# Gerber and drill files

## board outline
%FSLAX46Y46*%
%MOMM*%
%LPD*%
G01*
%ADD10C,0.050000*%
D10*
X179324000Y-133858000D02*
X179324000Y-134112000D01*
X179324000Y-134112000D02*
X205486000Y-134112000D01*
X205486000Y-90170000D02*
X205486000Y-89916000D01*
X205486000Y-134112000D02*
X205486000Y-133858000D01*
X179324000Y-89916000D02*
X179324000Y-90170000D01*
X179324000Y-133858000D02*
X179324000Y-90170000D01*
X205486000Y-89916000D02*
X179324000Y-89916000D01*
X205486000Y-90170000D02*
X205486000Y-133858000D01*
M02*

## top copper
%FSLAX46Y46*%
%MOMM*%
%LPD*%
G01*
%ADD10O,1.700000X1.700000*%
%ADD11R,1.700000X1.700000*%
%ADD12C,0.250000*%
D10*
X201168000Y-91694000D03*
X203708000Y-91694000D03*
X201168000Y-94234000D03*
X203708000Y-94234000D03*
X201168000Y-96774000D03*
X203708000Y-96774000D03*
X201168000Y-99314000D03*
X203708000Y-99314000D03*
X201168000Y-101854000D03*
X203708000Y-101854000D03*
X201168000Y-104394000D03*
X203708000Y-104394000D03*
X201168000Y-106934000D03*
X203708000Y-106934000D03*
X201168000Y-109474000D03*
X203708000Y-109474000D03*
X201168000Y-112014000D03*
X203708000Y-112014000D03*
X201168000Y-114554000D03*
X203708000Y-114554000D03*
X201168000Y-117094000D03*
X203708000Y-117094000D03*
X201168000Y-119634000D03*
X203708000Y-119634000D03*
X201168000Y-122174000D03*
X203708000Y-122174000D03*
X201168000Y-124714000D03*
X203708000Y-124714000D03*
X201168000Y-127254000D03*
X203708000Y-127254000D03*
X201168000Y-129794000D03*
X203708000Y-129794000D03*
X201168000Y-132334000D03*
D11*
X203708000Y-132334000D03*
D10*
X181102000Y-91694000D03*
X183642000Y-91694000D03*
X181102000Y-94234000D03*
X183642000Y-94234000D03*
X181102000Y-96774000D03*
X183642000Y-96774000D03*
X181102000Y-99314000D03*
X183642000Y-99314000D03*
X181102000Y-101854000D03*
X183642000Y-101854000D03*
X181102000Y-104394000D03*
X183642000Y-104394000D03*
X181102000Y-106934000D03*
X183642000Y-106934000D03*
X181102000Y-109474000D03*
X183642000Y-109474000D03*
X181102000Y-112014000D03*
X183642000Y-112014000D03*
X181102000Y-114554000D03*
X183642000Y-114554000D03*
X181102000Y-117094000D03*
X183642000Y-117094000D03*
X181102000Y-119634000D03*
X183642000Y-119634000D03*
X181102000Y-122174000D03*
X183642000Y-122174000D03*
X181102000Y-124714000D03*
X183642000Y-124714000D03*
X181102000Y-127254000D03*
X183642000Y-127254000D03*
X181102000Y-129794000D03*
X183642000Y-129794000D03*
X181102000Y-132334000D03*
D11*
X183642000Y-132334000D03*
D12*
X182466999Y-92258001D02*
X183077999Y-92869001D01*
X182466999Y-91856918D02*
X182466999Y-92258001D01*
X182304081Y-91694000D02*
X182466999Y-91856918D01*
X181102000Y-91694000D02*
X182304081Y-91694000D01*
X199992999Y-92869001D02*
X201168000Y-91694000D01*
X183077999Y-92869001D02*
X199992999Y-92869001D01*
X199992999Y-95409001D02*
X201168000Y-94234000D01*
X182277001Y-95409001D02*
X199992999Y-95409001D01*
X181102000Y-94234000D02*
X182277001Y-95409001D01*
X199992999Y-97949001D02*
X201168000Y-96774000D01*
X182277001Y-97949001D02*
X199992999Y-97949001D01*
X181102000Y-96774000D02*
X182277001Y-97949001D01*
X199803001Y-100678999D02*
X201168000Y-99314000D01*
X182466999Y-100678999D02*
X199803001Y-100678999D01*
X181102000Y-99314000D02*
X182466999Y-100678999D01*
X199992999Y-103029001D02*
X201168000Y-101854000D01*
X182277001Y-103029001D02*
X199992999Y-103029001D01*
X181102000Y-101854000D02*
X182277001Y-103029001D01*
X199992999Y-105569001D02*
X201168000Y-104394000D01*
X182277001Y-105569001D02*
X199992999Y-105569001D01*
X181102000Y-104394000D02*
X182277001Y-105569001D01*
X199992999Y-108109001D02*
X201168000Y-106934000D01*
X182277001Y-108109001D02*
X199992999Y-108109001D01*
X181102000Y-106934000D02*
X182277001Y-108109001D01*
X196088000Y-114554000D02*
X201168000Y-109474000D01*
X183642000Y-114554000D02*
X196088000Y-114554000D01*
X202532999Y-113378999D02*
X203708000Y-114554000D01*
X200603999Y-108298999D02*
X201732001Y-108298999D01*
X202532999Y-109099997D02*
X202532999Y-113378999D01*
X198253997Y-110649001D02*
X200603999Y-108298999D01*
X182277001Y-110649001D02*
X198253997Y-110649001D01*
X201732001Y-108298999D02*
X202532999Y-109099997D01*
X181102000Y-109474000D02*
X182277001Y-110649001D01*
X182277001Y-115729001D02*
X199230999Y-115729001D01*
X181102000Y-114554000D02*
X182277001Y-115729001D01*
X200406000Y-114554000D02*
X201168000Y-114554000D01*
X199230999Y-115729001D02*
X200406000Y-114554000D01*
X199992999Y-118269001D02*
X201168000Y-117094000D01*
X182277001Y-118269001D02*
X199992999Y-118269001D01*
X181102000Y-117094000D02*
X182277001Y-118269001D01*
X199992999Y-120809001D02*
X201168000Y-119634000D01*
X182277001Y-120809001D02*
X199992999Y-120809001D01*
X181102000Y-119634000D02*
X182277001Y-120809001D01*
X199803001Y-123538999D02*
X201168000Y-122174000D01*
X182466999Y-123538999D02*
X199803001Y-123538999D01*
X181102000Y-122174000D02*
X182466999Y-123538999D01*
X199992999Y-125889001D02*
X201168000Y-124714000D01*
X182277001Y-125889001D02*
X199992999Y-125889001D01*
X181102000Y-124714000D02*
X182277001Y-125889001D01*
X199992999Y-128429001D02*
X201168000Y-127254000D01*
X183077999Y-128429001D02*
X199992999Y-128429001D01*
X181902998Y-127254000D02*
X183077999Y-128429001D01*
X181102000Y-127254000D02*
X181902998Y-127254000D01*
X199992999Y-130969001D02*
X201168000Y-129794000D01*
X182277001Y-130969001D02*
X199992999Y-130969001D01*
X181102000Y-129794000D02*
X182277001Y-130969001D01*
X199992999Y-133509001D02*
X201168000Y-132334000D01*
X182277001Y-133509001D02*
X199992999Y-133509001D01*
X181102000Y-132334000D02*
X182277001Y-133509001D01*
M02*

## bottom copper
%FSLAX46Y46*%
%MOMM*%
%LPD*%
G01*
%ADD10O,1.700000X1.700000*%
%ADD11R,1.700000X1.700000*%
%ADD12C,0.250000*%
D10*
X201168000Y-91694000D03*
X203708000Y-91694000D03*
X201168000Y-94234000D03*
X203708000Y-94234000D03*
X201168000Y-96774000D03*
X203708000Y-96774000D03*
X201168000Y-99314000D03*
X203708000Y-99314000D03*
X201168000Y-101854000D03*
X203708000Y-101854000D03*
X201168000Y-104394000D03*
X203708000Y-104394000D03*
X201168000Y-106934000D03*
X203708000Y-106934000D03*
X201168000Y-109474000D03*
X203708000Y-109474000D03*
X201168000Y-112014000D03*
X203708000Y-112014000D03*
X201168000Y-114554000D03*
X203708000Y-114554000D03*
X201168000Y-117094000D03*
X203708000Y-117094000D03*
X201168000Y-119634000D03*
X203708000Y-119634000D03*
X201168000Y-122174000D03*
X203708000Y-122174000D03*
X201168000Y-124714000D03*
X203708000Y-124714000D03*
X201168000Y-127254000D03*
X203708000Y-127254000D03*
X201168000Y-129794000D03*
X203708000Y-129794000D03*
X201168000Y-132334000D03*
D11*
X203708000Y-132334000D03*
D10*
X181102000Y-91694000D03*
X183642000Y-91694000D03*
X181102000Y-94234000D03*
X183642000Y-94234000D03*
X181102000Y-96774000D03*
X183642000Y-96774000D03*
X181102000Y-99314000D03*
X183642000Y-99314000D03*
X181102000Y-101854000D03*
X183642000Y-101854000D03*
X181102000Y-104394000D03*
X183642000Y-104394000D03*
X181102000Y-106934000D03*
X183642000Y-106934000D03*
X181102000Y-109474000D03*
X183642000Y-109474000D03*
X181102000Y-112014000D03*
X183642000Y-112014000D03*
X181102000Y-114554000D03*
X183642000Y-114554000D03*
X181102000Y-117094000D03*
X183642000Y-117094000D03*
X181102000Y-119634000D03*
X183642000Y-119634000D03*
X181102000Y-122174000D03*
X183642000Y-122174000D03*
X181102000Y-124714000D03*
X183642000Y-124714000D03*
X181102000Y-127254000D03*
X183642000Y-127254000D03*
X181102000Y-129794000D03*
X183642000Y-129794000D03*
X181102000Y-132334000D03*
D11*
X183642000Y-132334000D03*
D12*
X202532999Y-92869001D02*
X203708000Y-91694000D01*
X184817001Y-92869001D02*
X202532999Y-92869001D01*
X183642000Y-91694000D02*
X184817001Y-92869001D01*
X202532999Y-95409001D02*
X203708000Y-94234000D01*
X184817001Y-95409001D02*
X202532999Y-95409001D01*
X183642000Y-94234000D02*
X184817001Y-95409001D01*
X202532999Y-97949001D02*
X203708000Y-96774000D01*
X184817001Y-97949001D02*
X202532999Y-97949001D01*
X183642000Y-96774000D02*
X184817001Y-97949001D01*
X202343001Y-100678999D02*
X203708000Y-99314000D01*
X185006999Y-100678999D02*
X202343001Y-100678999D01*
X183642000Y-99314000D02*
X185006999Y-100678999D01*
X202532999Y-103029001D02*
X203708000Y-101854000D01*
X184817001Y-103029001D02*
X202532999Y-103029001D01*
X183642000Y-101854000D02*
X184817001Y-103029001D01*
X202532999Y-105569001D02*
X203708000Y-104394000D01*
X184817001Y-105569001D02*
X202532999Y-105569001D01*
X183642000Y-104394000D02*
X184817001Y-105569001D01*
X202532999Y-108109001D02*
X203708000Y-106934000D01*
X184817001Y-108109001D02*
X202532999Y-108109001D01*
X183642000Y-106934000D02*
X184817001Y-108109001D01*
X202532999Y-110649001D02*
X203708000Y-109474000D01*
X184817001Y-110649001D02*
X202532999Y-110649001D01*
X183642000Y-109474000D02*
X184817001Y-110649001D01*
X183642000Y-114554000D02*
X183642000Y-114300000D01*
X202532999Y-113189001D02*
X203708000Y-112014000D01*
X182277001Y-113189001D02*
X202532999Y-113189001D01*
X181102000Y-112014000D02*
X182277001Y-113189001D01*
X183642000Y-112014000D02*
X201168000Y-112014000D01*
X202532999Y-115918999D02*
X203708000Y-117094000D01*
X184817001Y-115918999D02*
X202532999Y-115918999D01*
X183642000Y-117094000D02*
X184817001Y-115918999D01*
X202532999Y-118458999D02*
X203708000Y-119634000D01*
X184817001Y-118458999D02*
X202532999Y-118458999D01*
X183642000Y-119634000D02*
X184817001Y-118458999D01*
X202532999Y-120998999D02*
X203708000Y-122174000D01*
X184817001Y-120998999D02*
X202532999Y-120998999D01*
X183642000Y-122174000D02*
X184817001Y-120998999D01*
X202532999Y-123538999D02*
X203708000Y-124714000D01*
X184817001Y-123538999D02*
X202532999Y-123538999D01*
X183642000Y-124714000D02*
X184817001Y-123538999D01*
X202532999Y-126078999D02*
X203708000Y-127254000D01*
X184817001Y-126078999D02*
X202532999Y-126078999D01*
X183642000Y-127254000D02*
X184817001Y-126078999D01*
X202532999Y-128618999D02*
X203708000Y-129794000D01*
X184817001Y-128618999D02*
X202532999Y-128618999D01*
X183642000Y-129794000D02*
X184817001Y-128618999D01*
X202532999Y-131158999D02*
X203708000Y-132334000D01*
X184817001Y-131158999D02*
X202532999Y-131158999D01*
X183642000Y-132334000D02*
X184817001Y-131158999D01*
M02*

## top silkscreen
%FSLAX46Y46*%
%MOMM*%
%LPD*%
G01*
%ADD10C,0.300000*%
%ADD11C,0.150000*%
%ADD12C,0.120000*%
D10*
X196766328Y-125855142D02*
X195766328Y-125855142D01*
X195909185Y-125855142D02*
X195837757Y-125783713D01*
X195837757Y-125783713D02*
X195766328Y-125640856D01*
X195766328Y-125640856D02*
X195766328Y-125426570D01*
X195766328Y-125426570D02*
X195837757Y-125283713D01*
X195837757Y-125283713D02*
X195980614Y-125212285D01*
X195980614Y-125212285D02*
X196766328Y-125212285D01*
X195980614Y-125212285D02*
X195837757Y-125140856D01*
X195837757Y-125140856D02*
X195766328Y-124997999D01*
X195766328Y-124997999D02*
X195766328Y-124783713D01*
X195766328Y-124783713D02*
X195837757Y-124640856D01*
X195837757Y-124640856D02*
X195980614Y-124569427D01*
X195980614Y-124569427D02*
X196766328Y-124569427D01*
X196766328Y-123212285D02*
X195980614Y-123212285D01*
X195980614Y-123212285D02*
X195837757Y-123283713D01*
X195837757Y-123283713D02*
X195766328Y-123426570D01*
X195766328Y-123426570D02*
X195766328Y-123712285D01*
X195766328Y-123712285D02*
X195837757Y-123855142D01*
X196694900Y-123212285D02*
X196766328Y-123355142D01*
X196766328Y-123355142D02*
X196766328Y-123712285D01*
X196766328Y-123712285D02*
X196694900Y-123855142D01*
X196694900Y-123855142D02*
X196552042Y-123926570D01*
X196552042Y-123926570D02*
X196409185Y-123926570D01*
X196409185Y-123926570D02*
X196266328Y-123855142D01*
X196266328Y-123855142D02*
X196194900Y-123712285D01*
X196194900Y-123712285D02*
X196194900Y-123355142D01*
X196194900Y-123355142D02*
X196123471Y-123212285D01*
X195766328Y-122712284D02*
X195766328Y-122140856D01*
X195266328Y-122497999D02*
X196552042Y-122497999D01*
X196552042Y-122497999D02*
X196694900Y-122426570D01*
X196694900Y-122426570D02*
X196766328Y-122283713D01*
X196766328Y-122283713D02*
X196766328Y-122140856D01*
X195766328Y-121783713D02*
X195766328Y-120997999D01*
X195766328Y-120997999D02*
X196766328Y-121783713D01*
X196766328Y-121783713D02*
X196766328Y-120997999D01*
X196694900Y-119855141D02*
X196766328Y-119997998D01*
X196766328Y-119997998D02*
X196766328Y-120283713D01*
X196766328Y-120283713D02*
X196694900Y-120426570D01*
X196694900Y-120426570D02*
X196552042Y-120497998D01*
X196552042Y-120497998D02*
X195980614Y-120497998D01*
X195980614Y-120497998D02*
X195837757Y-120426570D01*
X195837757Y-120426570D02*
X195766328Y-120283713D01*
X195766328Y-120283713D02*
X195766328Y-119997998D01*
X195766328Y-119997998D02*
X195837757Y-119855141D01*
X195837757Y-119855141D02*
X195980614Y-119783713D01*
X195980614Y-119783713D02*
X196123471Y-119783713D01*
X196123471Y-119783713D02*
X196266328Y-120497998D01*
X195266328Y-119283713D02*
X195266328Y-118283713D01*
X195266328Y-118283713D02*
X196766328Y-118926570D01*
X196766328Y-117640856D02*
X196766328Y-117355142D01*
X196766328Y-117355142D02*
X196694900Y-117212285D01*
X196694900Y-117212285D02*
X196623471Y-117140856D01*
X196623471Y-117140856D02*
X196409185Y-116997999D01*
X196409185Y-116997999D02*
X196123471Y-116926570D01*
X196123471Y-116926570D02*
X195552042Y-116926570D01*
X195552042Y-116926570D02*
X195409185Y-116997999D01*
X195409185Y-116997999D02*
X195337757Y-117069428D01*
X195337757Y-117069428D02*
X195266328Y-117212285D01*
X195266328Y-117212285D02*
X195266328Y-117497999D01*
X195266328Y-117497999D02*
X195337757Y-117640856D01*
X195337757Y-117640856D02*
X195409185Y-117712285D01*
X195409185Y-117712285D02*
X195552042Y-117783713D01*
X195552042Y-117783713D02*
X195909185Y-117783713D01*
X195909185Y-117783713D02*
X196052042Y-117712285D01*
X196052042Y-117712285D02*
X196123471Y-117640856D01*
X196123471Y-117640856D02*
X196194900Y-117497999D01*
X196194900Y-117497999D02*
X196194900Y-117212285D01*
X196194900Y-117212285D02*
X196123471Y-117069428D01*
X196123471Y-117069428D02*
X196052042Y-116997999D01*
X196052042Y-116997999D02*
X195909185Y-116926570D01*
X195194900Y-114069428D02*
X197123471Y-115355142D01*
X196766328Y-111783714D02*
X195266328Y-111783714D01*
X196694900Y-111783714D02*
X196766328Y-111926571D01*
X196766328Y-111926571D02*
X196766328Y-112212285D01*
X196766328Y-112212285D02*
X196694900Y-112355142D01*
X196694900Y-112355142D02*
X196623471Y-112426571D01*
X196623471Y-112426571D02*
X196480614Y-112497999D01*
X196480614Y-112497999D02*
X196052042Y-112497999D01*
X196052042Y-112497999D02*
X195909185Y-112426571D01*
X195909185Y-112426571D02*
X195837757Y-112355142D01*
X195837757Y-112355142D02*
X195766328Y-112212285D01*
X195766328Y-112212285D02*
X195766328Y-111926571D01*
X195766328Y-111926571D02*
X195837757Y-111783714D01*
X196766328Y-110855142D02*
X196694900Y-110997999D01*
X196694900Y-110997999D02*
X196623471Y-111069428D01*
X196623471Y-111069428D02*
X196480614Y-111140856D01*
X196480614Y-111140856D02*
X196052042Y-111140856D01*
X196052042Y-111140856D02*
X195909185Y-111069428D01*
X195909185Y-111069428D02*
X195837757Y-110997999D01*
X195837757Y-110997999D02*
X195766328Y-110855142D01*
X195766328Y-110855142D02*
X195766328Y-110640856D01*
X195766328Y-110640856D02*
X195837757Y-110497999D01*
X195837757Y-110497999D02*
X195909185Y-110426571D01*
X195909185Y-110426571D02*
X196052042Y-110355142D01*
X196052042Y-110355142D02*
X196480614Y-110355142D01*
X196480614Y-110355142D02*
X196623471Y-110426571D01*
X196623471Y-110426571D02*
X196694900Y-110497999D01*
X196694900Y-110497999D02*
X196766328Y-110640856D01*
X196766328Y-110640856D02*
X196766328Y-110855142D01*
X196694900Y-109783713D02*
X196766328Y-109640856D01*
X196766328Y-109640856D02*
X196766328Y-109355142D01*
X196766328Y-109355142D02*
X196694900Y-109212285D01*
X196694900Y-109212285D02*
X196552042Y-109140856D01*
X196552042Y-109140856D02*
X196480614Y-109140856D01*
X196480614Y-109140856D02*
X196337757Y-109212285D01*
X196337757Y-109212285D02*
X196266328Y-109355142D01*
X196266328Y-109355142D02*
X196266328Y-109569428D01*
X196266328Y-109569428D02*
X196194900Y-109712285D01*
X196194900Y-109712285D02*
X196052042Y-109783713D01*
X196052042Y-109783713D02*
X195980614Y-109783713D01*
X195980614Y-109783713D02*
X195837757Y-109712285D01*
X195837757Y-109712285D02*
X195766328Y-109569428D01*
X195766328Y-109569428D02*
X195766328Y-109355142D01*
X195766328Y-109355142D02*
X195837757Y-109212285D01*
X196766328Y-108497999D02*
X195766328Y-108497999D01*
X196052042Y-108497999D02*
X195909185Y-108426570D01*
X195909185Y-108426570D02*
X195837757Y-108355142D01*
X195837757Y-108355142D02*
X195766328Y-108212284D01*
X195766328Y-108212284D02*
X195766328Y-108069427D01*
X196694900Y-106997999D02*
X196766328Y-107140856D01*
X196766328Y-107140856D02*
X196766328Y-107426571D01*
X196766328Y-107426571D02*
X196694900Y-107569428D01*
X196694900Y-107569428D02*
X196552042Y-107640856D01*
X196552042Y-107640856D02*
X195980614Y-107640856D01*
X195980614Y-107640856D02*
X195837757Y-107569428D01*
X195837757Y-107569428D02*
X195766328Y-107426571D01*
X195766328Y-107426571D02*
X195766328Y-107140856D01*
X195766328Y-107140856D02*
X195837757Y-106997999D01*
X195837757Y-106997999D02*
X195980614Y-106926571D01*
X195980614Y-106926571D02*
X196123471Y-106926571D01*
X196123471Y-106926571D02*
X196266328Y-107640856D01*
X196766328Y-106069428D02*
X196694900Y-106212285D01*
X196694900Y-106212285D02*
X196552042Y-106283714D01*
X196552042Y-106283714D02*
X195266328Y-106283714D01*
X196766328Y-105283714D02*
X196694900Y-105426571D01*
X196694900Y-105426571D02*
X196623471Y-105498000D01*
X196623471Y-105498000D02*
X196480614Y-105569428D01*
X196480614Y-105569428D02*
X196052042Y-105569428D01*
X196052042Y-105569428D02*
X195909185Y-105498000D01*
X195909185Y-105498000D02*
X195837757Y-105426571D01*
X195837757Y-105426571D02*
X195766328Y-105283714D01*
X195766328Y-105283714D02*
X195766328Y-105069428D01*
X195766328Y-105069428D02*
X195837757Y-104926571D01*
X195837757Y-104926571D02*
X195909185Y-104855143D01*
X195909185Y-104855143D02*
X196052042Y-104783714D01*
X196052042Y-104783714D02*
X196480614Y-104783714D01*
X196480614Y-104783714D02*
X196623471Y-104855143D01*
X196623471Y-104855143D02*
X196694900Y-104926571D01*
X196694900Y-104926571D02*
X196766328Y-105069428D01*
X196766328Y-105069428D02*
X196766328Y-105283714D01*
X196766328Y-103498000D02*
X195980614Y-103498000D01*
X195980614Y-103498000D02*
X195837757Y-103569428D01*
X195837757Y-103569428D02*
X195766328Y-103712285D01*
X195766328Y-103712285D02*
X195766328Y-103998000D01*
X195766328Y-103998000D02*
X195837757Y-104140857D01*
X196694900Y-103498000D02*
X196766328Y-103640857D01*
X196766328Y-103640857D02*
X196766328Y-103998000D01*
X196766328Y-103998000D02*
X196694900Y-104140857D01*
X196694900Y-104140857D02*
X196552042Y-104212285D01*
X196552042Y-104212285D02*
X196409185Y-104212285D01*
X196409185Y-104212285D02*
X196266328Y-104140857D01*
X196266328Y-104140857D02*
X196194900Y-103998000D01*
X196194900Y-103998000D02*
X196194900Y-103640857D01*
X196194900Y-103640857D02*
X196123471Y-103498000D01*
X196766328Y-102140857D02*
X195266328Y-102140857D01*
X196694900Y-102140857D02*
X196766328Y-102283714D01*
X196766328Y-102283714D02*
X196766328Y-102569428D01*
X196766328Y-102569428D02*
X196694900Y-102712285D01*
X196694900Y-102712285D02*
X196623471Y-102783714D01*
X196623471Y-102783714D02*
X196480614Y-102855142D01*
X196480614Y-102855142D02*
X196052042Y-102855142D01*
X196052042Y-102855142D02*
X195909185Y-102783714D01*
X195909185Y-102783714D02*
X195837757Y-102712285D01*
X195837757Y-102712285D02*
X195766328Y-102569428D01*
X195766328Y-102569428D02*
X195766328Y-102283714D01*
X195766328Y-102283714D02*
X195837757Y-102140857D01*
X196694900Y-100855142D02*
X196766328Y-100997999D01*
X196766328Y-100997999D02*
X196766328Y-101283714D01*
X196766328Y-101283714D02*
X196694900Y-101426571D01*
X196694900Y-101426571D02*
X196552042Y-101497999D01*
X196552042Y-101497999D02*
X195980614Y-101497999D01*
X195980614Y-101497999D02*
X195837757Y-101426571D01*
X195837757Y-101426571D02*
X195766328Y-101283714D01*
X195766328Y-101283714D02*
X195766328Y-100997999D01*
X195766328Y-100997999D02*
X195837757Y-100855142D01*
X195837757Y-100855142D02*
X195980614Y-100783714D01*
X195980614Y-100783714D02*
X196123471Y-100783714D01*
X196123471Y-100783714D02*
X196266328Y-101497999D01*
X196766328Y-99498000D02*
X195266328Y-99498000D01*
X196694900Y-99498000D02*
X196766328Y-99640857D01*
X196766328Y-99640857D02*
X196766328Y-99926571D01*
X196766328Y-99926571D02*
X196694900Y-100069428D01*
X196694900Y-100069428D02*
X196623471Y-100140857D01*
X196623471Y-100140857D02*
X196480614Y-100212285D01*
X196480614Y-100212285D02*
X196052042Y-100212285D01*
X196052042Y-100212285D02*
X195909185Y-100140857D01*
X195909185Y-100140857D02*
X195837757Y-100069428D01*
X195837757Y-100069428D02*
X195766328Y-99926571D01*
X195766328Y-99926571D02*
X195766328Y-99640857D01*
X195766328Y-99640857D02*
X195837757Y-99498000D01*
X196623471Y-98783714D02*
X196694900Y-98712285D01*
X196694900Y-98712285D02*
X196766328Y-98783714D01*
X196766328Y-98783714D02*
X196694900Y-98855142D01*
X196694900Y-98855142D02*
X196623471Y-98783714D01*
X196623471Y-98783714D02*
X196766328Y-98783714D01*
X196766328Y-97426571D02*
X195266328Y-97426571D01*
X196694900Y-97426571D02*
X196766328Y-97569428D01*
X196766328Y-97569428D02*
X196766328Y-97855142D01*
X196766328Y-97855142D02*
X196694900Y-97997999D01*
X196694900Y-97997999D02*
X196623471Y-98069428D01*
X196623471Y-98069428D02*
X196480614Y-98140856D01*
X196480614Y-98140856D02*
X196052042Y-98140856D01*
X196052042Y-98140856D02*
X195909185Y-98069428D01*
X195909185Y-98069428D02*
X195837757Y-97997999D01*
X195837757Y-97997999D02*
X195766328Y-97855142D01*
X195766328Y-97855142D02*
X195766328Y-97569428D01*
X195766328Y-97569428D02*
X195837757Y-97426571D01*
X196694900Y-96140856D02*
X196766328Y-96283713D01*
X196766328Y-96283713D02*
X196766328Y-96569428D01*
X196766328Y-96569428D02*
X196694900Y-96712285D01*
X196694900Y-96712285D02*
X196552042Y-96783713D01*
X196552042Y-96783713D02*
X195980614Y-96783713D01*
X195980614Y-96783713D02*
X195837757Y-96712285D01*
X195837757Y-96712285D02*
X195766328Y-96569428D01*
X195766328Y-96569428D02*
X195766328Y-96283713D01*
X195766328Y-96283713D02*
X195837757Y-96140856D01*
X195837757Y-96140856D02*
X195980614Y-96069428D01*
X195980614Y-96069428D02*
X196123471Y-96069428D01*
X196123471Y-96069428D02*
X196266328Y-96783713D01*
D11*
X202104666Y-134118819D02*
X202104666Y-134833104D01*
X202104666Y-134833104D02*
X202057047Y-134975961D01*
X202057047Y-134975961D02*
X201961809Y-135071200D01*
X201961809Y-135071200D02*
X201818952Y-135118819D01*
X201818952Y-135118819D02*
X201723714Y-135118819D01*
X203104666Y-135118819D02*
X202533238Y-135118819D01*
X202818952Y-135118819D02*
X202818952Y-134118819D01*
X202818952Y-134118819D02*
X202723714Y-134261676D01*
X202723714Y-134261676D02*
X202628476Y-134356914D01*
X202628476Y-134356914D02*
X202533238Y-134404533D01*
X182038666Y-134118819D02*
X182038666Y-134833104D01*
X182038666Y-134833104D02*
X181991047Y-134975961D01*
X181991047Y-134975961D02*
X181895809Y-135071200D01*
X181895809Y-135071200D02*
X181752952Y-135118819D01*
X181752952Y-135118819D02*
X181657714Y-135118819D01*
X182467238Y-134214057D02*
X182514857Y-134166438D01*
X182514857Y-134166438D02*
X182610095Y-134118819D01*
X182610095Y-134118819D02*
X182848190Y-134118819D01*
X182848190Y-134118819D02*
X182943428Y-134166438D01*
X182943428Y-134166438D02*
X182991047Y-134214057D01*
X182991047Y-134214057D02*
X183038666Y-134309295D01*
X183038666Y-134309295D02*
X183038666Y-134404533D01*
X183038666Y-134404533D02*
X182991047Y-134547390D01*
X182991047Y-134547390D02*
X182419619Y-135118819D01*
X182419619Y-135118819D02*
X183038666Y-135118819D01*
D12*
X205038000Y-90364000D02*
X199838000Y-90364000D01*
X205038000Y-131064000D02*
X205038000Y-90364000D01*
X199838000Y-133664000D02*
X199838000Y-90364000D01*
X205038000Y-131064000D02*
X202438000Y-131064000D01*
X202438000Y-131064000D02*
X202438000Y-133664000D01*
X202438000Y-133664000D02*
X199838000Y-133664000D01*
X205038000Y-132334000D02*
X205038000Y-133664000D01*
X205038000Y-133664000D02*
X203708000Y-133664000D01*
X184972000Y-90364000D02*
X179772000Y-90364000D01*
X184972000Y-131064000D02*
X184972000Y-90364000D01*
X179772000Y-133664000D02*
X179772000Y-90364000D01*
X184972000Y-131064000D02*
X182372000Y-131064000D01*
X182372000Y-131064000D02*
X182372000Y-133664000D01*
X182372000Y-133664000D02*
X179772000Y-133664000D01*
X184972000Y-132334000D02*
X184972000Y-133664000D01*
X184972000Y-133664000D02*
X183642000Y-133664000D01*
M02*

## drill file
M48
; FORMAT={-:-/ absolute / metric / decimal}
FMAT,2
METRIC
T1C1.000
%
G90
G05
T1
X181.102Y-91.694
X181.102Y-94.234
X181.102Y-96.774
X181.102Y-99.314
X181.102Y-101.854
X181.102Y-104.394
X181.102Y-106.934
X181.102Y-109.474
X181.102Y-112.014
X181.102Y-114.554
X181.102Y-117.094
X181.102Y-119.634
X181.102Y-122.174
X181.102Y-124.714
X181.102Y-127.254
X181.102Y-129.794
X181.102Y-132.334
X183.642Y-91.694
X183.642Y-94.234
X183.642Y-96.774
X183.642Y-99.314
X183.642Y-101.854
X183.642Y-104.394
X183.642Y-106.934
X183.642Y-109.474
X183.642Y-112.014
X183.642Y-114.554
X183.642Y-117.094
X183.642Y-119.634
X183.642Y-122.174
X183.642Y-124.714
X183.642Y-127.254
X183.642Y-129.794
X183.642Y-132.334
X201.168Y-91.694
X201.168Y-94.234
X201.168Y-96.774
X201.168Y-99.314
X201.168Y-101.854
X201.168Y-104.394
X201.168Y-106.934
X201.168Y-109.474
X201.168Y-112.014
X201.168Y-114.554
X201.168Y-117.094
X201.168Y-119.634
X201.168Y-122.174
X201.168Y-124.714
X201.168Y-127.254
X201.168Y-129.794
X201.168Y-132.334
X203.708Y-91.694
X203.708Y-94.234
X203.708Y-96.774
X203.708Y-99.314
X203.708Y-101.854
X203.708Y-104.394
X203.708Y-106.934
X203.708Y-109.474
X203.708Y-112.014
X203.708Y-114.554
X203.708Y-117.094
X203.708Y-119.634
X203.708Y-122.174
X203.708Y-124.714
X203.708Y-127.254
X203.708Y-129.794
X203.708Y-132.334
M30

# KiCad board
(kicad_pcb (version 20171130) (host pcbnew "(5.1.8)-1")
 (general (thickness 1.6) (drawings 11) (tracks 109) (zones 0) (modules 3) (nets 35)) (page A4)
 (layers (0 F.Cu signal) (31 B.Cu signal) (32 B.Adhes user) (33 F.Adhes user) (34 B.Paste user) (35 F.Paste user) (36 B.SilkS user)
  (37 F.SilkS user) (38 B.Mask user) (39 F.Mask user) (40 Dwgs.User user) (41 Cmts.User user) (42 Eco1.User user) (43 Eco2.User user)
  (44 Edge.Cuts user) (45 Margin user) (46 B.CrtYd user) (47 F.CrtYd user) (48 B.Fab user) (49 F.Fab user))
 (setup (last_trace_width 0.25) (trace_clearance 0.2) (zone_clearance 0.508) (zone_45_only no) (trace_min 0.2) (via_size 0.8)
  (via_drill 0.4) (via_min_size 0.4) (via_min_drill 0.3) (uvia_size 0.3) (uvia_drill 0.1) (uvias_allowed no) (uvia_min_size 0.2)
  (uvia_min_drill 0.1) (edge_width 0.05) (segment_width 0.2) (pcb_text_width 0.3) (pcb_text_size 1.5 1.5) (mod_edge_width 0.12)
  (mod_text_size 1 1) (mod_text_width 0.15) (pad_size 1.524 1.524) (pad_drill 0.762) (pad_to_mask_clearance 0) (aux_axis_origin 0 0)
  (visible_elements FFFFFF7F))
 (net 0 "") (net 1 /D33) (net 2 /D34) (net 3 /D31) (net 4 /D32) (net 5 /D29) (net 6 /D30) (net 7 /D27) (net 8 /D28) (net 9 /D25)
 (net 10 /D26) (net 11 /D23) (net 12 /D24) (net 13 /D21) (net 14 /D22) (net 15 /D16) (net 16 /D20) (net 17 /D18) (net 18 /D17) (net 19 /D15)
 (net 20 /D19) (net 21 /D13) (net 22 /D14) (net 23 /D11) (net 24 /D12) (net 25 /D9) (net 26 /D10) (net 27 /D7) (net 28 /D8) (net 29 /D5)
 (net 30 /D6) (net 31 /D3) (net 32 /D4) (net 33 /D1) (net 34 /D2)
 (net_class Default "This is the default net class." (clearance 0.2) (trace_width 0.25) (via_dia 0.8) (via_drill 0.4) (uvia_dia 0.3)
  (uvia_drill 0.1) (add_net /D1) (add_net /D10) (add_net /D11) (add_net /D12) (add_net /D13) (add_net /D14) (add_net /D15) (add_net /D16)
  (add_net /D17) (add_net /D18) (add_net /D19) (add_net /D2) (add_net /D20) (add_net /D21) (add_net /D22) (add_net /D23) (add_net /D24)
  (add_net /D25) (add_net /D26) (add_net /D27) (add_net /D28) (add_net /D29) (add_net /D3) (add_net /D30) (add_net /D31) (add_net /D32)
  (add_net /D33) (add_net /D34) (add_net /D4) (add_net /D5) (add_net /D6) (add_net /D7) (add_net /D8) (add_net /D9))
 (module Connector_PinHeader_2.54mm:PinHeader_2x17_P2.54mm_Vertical (layer F.Cu) (at 203.708 132.334 180)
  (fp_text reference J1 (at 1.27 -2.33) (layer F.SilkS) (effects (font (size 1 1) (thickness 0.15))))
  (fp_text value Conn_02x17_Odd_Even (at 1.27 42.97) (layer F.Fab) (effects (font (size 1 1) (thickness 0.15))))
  (fp_line (start -1.33 41.97) (end 3.87 41.97) (layer F.SilkS) (width 0.12))
  (fp_line (start -1.33 1.27) (end -1.33 41.97) (layer F.SilkS) (width 0.12))
  (fp_line (start 3.87 -1.33) (end 3.87 41.97) (layer F.SilkS) (width 0.12))
  (fp_line (start -1.33 1.27) (end 1.27 1.27) (layer F.SilkS) (width 0.12))
  (fp_line (start 1.27 1.27) (end 1.27 -1.33) (layer F.SilkS) (width 0.12))
  (fp_line (start 1.27 -1.33) (end 3.87 -1.33) (layer F.SilkS) (width 0.12))
  (fp_line (start -1.33 0) (end -1.33 -1.33) (layer F.SilkS) (width 0.12))
  (fp_line (start -1.33 -1.33) (end 0 -1.33) (layer F.SilkS) (width 0.12))
  (pad 34 thru_hole oval (at 2.54 40.64 180) (size 1.7 1.7) (drill 1) (layers *.Cu *.Mask) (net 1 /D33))
  (pad 33 thru_hole oval (at 0 40.64 180) (size 1.7 1.7) (drill 1) (layers *.Cu *.Mask) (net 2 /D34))
  (pad 32 thru_hole oval (at 2.54 38.1 180) (size 1.7 1.7) (drill 1) (layers *.Cu *.Mask) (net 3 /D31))
  (pad 31 thru_hole oval (at 0 38.1 180) (size 1.7 1.7) (drill 1) (layers *.Cu *.Mask) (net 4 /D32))
  (pad 30 thru_hole oval (at 2.54 35.56 180) (size 1.7 1.7) (drill 1) (layers *.Cu *.Mask) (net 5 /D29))
  (pad 29 thru_hole oval (at 0 35.56 180) (size 1.7 1.7) (drill 1) (layers *.Cu *.Mask) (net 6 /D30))
  (pad 28 thru_hole oval (at 2.54 33.02 180) (size 1.7 1.7) (drill 1) (layers *.Cu *.Mask) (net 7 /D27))
  (pad 27 thru_hole oval (at 0 33.02 180) (size 1.7 1.7) (drill 1) (layers *.Cu *.Mask) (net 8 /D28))
  (pad 26 thru_hole oval (at 2.54 30.48 180) (size 1.7 1.7) (drill 1) (layers *.Cu *.Mask) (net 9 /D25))
  (pad 25 thru_hole oval (at 0 30.48 180) (size 1.7 1.7) (drill 1) (layers *.Cu *.Mask) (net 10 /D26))
  (pad 24 thru_hole oval (at 2.54 27.94 180) (size 1.7 1.7) (drill 1) (layers *.Cu *.Mask) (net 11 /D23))
  (pad 23 thru_hole oval (at 0 27.94 180) (size 1.7 1.7) (drill 1) (layers *.Cu *.Mask) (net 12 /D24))
  (pad 22 thru_hole oval (at 2.54 25.4 180) (size 1.7 1.7) (drill 1) (layers *.Cu *.Mask) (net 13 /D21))
  (pad 21 thru_hole oval (at 0 25.4 180) (size 1.7 1.7) (drill 1) (layers *.Cu *.Mask) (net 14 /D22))
  (pad 20 thru_hole oval (at 2.54 22.86 180) (size 1.7 1.7) (drill 1) (layers *.Cu *.Mask) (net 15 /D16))
  (pad 19 thru_hole oval (at 0 22.86 180) (size 1.7 1.7) (drill 1) (layers *.Cu *.Mask) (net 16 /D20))
  (pad 18 thru_hole oval (at 2.54 20.32 180) (size 1.7 1.7) (drill 1) (layers *.Cu *.Mask) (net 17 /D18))
  (pad 17 thru_hole oval (at 0 20.32 180) (size 1.7 1.7) (drill 1) (layers *.Cu *.Mask) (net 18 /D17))
  (pad 16 thru_hole oval (at 2.54 17.78 180) (size 1.7 1.7) (drill 1) (layers *.Cu *.Mask) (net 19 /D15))
  (pad 15 thru_hole oval (at 0 17.78 180) (size 1.7 1.7) (drill 1) (layers *.Cu *.Mask) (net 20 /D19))
  (pad 14 thru_hole oval (at 2.54 15.24 180) (size 1.7 1.7) (drill 1) (layers *.Cu *.Mask) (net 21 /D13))
  (pad 13 thru_hole oval (at 0 15.24 180) (size 1.7 1.7) (drill 1) (layers *.Cu *.Mask) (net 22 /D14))
  (pad 12 thru_hole oval (at 2.54 12.7 180) (size 1.7 1.7) (drill 1) (layers *.Cu *.Mask) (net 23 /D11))
  (pad 11 thru_hole oval (at 0 12.7 180) (size 1.7 1.7) (drill 1) (layers *.Cu *.Mask) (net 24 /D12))
  (pad 10 thru_hole oval (at 2.54 10.16 180) (size 1.7 1.7) (drill 1) (layers *.Cu *.Mask) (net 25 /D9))
  (pad 9 thru_hole oval (at 0 10.16 180) (size 1.7 1.7) (drill 1) (layers *.Cu *.Mask) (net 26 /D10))
  (pad 8 thru_hole oval (at 2.54 7.62 180) (size 1.7 1.7) (drill 1) (layers *.Cu *.Mask) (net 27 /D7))
  (pad 7 thru_hole oval (at 0 7.62 180) (size 1.7 1.7) (drill 1) (layers *.Cu *.Mask) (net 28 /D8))
  (pad 6 thru_hole oval (at 2.54 5.08 180) (size 1.7 1.7) (drill 1) (layers *.Cu *.Mask) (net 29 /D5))
  (pad 5 thru_hole oval (at 0 5.08 180) (size 1.7 1.7) (drill 1) (layers *.Cu *.Mask) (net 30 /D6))
  (pad 4 thru_hole oval (at 2.54 2.54 180) (size 1.7 1.7) (drill 1) (layers *.Cu *.Mask) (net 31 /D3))
  (pad 3 thru_hole oval (at 0 2.54 180) (size 1.7 1.7) (drill 1) (layers *.Cu *.Mask) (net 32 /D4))
  (pad 2 thru_hole oval (at 2.54 0 180) (size 1.7 1.7) (drill 1) (layers *.Cu *.Mask) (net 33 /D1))
  (pad 1 thru_hole rect (at 0 0 180) (size 1.7 1.7) (drill 1) (layers *.Cu *.Mask) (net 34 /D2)))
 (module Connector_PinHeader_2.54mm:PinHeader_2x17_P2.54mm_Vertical (layer F.Cu) (at 183.642 132.334 180)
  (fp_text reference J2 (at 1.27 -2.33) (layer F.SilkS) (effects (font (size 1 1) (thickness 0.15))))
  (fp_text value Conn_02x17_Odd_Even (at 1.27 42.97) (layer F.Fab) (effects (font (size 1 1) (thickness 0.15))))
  (fp_line (start -1.33 41.97) (end 3.87 41.97) (layer F.SilkS) (width 0.12))
  (fp_line (start -1.33 1.27) (end -1.33 41.97) (layer F.SilkS) (width 0.12))
  (fp_line (start 3.87 -1.33) (end 3.87 41.97) (layer F.SilkS) (width 0.12))
  (fp_line (start -1.33 1.27) (end 1.27 1.27) (layer F.SilkS) (width 0.12))
  (fp_line (start 1.27 1.27) (end 1.27 -1.33) (layer F.SilkS) (width 0.12))
  (fp_line (start 1.27 -1.33) (end 3.87 -1.33) (layer F.SilkS) (width 0.12))
  (fp_line (start -1.33 0) (end -1.33 -1.33) (layer F.SilkS) (width 0.12))
  (fp_line (start -1.33 -1.33) (end 0 -1.33) (layer F.SilkS) (width 0.12))
  (pad 34 thru_hole oval (at 2.54 40.64 180) (size 1.7 1.7) (drill 1) (layers *.Cu *.Mask) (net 1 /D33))
  (pad 33 thru_hole oval (at 0 40.64 180) (size 1.7 1.7) (drill 1) (layers *.Cu *.Mask) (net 2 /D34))
  (pad 32 thru_hole oval (at 2.54 38.1 180) (size 1.7 1.7) (drill 1) (layers *.Cu *.Mask) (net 3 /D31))
  (pad 31 thru_hole oval (at 0 38.1 180) (size 1.7 1.7) (drill 1) (layers *.Cu *.Mask) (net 4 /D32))
  (pad 30 thru_hole oval (at 2.54 35.56 180) (size 1.7 1.7) (drill 1) (layers *.Cu *.Mask) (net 5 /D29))
  (pad 29 thru_hole oval (at 0 35.56 180) (size 1.7 1.7) (drill 1) (layers *.Cu *.Mask) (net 6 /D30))
  (pad 28 thru_hole oval (at 2.54 33.02 180) (size 1.7 1.7) (drill 1) (layers *.Cu *.Mask) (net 7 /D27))
  (pad 27 thru_hole oval (at 0 33.02 180) (size 1.7 1.7) (drill 1) (layers *.Cu *.Mask) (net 8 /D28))
  (pad 26 thru_hole oval (at 2.54 30.48 180) (size 1.7 1.7) (drill 1) (layers *.Cu *.Mask) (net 9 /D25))
  (pad 25 thru_hole oval (at 0 30.48 180) (size 1.7 1.7) (drill 1) (layers *.Cu *.Mask) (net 10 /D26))
  (pad 24 thru_hole oval (at 2.54 27.94 180) (size 1.7 1.7) (drill 1) (layers *.Cu *.Mask) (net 11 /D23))
  (pad 23 thru_hole oval (at 0 27.94 180) (size 1.7 1.7) (drill 1) (layers *.Cu *.Mask) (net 12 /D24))
  (pad 22 thru_hole oval (at 2.54 25.4 180) (size 1.7 1.7) (drill 1) (layers *.Cu *.Mask) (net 13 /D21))
  (pad 21 thru_hole oval (at 0 25.4 180) (size 1.7 1.7) (drill 1) (layers *.Cu *.Mask) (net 14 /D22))
  (pad 20 thru_hole oval (at 2.54 22.86 180) (size 1.7 1.7) (drill 1) (layers *.Cu *.Mask) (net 20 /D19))
  (pad 19 thru_hole oval (at 0 22.86 180) (size 1.7 1.7) (drill 1) (layers *.Cu *.Mask) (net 16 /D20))
  (pad 18 thru_hole oval (at 2.54 20.32 180) (size 1.7 1.7) (drill 1) (layers *.Cu *.Mask) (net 18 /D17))
  (pad 17 thru_hole oval (at 0 20.32 180) (size 1.7 1.7) (drill 1) (layers *.Cu *.Mask) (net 17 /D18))
  (pad 16 thru_hole oval (at 2.54 17.78 180) (size 1.7 1.7) (drill 1) (layers *.Cu *.Mask) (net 19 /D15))
  (pad 15 thru_hole oval (at 0 17.78 180) (size 1.7 1.7) (drill 1) (layers *.Cu *.Mask) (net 15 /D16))
  (pad 14 thru_hole oval (at 2.54 15.24 180) (size 1.7 1.7) (drill 1) (layers *.Cu *.Mask) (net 21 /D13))
  (pad 13 thru_hole oval (at 0 15.24 180) (size 1.7 1.7) (drill 1) (layers *.Cu *.Mask) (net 22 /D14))
  (pad 12 thru_hole oval (at 2.54 12.7 180) (size 1.7 1.7) (drill 1) (layers *.Cu *.Mask) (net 23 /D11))
  (pad 11 thru_hole oval (at 0 12.7 180) (size 1.7 1.7) (drill 1) (layers *.Cu *.Mask) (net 24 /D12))
  (pad 10 thru_hole oval (at 2.54 10.16 180) (size 1.7 1.7) (drill 1) (layers *.Cu *.Mask) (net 25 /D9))
  (pad 9 thru_hole oval (at 0 10.16 180) (size 1.7 1.7) (drill 1) (layers *.Cu *.Mask) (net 26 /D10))
  (pad 8 thru_hole oval (at 2.54 7.62 180) (size 1.7 1.7) (drill 1) (layers *.Cu *.Mask) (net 27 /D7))
  (pad 7 thru_hole oval (at 0 7.62 180) (size 1.7 1.7) (drill 1) (layers *.Cu *.Mask) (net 28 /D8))
  (pad 6 thru_hole oval (at 2.54 5.08 180) (size 1.7 1.7) (drill 1) (layers *.Cu *.Mask) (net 29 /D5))
  (pad 5 thru_hole oval (at 0 5.08 180) (size 1.7 1.7) (drill 1) (layers *.Cu *.Mask) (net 30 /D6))
  (pad 4 thru_hole oval (at 2.54 2.54 180) (size 1.7 1.7) (drill 1) (layers *.Cu *.Mask) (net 31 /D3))
  (pad 3 thru_hole oval (at 0 2.54 180) (size 1.7 1.7) (drill 1) (layers *.Cu *.Mask) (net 32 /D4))
  (pad 2 thru_hole oval (at 2.54 0 180) (size 1.7 1.7) (drill 1) (layers *.Cu *.Mask) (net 33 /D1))
  (pad 1 thru_hole rect (at 0 0 180) (size 1.7 1.7) (drill 1) (layers *.Cu *.Mask) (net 34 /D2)))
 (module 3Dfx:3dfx (layer B.Cu) (at 192.278 112.522 270)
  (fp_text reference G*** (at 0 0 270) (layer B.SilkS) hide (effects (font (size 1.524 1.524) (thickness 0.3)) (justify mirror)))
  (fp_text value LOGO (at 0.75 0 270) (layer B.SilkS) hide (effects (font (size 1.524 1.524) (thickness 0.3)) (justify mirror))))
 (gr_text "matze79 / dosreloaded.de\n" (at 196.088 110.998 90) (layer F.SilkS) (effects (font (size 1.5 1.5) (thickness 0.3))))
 (gr_line (start 179.324 133.858) (end 179.324 134.112) (layer Edge.Cuts) (width 0.05))
 (gr_line (start 179.324 134.112) (end 205.486 134.112) (layer Edge.Cuts) (width 0.05))
 (gr_line (start 205.486 90.17) (end 205.486 89.916) (layer Edge.Cuts) (width 0.05))
 (gr_line (start 205.486 134.112) (end 205.486 133.858) (layer Edge.Cuts) (width 0.05))
 (gr_line (start 179.324 89.916) (end 179.324 90.17) (layer Edge.Cuts) (width 0.05))
 (gr_line (start 179.324 133.858) (end 179.324 90.17) (layer Edge.Cuts) (width 0.05))
 (gr_line (start 205.486 89.916) (end 179.324 89.916) (layer Edge.Cuts) (width 0.05))
 (gr_line (start 205.486 90.17) (end 205.486 133.858) (layer Edge.Cuts) (width 0.05))
 (segment (start 202.532999 92.869001) (end 203.708 91.694) (width 0.25) (layer B.Cu) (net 2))
 (segment (start 184.817001 92.869001) (end 202.532999 92.869001) (width 0.25) (layer B.Cu) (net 2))
 (segment (start 183.642 91.694) (end 184.817001 92.869001) (width 0.25) (layer B.Cu) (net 2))
 (segment (start 182.466999 92.258001) (end 183.077999 92.869001) (width 0.25) (layer F.Cu) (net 1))
 (segment (start 182.466999 91.856918) (end 182.466999 92.258001) (width 0.25) (layer F.Cu) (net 1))
 (segment (start 182.304081 91.694) (end 182.466999 91.856918) (width 0.25) (layer F.Cu) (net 1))
 (segment (start 181.102 91.694) (end 182.304081 91.694) (width 0.25) (layer F.Cu) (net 1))
 (segment (start 199.992999 92.869001) (end 201.168 91.694) (width 0.25) (layer F.Cu) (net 1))
 (segment (start 183.077999 92.869001) (end 199.992999 92.869001) (width 0.25) (layer F.Cu) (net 1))
 (segment (start 202.532999 95.409001) (end 203.708 94.234) (width 0.25) (layer B.Cu) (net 4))
 (segment (start 184.817001 95.409001) (end 202.532999 95.409001) (width 0.25) (layer B.Cu) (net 4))
 (segment (start 183.642 94.234) (end 184.817001 95.409001) (width 0.25) (layer B.Cu) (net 4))
 (segment (start 199.992999 95.409001) (end 201.168 94.234) (width 0.25) (layer F.Cu) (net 3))
 (segment (start 182.277001 95.409001) (end 199.992999 95.409001) (width 0.25) (layer F.Cu) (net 3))
 (segment (start 181.102 94.234) (end 182.277001 95.409001) (width 0.25) (layer F.Cu) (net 3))
 (segment (start 202.532999 97.949001) (end 203.708 96.774) (width 0.25) (layer B.Cu) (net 6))
 (segment (start 184.817001 97.949001) (end 202.532999 97.949001) (width 0.25) (layer B.Cu) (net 6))
 (segment (start 183.642 96.774) (end 184.817001 97.949001) (width 0.25) (layer B.Cu) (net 6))
 (segment (start 199.992999 97.949001) (end 201.168 96.774) (width 0.25) (layer F.Cu) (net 5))
 (segment (start 182.277001 97.949001) (end 199.992999 97.949001) (width 0.25) (layer F.Cu) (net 5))
 (segment (start 181.102 96.774) (end 182.277001 97.949001) (width 0.25) (layer F.Cu) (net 5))
 (segment (start 202.343001 100.678999) (end 203.708 99.314) (width 0.25) (layer B.Cu) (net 8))
 (segment (start 185.006999 100.678999) (end 202.343001 100.678999) (width 0.25) (layer B.Cu) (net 8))
 (segment (start 183.642 99.314) (end 185.006999 100.678999) (width 0.25) (layer B.Cu) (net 8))
 (segment (start 199.803001 100.678999) (end 201.168 99.314) (width 0.25) (layer F.Cu) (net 7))
 (segment (start 182.466999 100.678999) (end 199.803001 100.678999) (width 0.25) (layer F.Cu) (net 7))
 (segment (start 181.102 99.314) (end 182.466999 100.678999) (width 0.25) (layer F.Cu) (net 7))
 (segment (start 202.532999 103.029001) (end 203.708 101.854) (width 0.25) (layer B.Cu) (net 10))
 (segment (start 184.817001 103.029001) (end 202.532999 103.029001) (width 0.25) (layer B.Cu) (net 10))
 (segment (start 183.642 101.854) (end 184.817001 103.029001) (width 0.25) (layer B.Cu) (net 10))
 (segment (start 199.992999 103.029001) (end 201.168 101.854) (width 0.25) (layer F.Cu) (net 9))
 (segment (start 182.277001 103.029001) (end 199.992999 103.029001) (width 0.25) (layer F.Cu) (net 9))
 (segment (start 181.102 101.854) (end 182.277001 103.029001) (width 0.25) (layer F.Cu) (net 9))
 (segment (start 202.532999 105.569001) (end 203.708 104.394) (width 0.25) (layer B.Cu) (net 12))
 (segment (start 184.817001 105.569001) (end 202.532999 105.569001) (width 0.25) (layer B.Cu) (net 12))
 (segment (start 183.642 104.394) (end 184.817001 105.569001) (width 0.25) (layer B.Cu) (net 12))
 (segment (start 199.992999 105.569001) (end 201.168 104.394) (width 0.25) (layer F.Cu) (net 11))
 (segment (start 182.277001 105.569001) (end 199.992999 105.569001) (width 0.25) (layer F.Cu) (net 11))
 (segment (start 181.102 104.394) (end 182.277001 105.569001) (width 0.25) (layer F.Cu) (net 11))
 (segment (start 202.532999 108.109001) (end 203.708 106.934) (width 0.25) (layer B.Cu) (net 14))
 (segment (start 184.817001 108.109001) (end 202.532999 108.109001) (width 0.25) (layer B.Cu) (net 14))
 (segment (start 183.642 106.934) (end 184.817001 108.109001) (width 0.25) (layer B.Cu) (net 14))
 (segment (start 199.992999 108.109001) (end 201.168 106.934) (width 0.25) (layer F.Cu) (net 13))
 (segment (start 182.277001 108.109001) (end 199.992999 108.109001) (width 0.25) (layer F.Cu) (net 13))
 (segment (start 181.102 106.934) (end 182.277001 108.109001) (width 0.25) (layer F.Cu) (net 13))
 (segment (start 202.532999 110.649001) (end 203.708 109.474) (width 0.25) (layer B.Cu) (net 16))
 (segment (start 184.817001 110.649001) (end 202.532999 110.649001) (width 0.25) (layer B.Cu) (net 16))
 (segment (start 183.642 109.474) (end 184.817001 110.649001) (width 0.25) (layer B.Cu) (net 16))
 (segment (start 183.642 114.554) (end 183.642 114.3) (width 0.25) (layer B.Cu) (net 15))
 (segment (start 196.088 114.554) (end 201.168 109.474) (width 0.25) (layer F.Cu) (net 15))
 (segment (start 183.642 114.554) (end 196.088 114.554) (width 0.25) (layer F.Cu) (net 15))
 (segment (start 202.532999 113.189001) (end 203.708 112.014) (width 0.25) (layer B.Cu) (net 18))
 (segment (start 182.277001 113.189001) (end 202.532999 113.189001) (width 0.25) (layer B.Cu) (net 18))
 (segment (start 181.102 112.014) (end 182.277001 113.189001) (width 0.25) (layer B.Cu) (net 18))
 (segment (start 183.642 112.014) (end 201.168 112.014) (width 0.25) (layer B.Cu) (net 17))
 (segment (start 202.532999 113.378999) (end 203.708 114.554) (width 0.25) (layer F.Cu) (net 20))
 (segment (start 200.603999 108.298999) (end 201.732001 108.298999) (width 0.25) (layer F.Cu) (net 20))
 (segment (start 202.532999 109.099997) (end 202.532999 113.378999) (width 0.25) (layer F.Cu) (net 20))
 (segment (start 198.253997 110.649001) (end 200.603999 108.298999) (width 0.25) (layer F.Cu) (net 20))
 (segment (start 182.277001 110.649001) (end 198.253997 110.649001) (width 0.25) (layer F.Cu) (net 20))
 (segment (start 201.732001 108.298999) (end 202.532999 109.099997) (width 0.25) (layer F.Cu) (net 20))
 (segment (start 181.102 109.474) (end 182.277001 110.649001) (width 0.25) (layer F.Cu) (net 20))
 (segment (start 182.277001 115.729001) (end 199.230999 115.729001) (width 0.25) (layer F.Cu) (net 19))
 (segment (start 181.102 114.554) (end 182.277001 115.729001) (width 0.25) (layer F.Cu) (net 19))
 (segment (start 200.406 114.554) (end 201.168 114.554) (width 0.25) (layer F.Cu) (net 19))
 (segment (start 199.230999 115.729001) (end 200.406 114.554) (width 0.25) (layer F.Cu) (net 19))
 (segment (start 202.532999 115.918999) (end 203.708 117.094) (width 0.25) (layer B.Cu) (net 22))
 (segment (start 184.817001 115.918999) (end 202.532999 115.918999) (width 0.25) (layer B.Cu) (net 22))
 (segment (start 183.642 117.094) (end 184.817001 115.918999) (width 0.25) (layer B.Cu) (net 22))
 (segment (start 199.992999 118.269001) (end 201.168 117.094) (width 0.25) (layer F.Cu) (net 21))
 (segment (start 182.277001 118.269001) (end 199.992999 118.269001) (width 0.25) (layer F.Cu) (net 21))
 (segment (start 181.102 117.094) (end 182.277001 118.269001) (width 0.25) (layer F.Cu) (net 21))
 (segment (start 202.532999 118.458999) (end 203.708 119.634) (width 0.25) (layer B.Cu) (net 24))
 (segment (start 184.817001 118.458999) (end 202.532999 118.458999) (width 0.25) (layer B.Cu) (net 24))
 (segment (start 183.642 119.634) (end 184.817001 118.458999) (width 0.25) (layer B.Cu) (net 24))
 (segment (start 199.992999 120.809001) (end 201.168 119.634) (width 0.25) (layer F.Cu) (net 23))
 (segment (start 182.277001 120.809001) (end 199.992999 120.809001) (width 0.25) (layer F.Cu) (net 23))
 (segment (start 181.102 119.634) (end 182.277001 120.809001) (width 0.25) (layer F.Cu) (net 23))
 (segment (start 202.532999 120.998999) (end 203.708 122.174) (width 0.25) (layer B.Cu) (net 26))
 (segment (start 184.817001 120.998999) (end 202.532999 120.998999) (width 0.25) (layer B.Cu) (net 26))
 (segment (start 183.642 122.174) (end 184.817001 120.998999) (width 0.25) (layer B.Cu) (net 26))
 (segment (start 199.803001 123.538999) (end 201.168 122.174) (width 0.25) (layer F.Cu) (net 25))
 (segment (start 182.466999 123.538999) (end 199.803001 123.538999) (width 0.25) (layer F.Cu) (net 25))
 (segment (start 181.102 122.174) (end 182.466999 123.538999) (width 0.25) (layer F.Cu) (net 25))
 (segment (start 202.532999 123.538999) (end 203.708 124.714) (width 0.25) (layer B.Cu) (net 28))
 (segment (start 184.817001 123.538999) (end 202.532999 123.538999) (width 0.25) (layer B.Cu) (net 28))
 (segment (start 183.642 124.714) (end 184.817001 123.538999) (width 0.25) (layer B.Cu) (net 28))
 (segment (start 199.992999 125.889001) (end 201.168 124.714) (width 0.25) (layer F.Cu) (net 27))
 (segment (start 182.277001 125.889001) (end 199.992999 125.889001) (width 0.25) (layer F.Cu) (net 27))
 (segment (start 181.102 124.714) (end 182.277001 125.889001) (width 0.25) (layer F.Cu) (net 27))
 (segment (start 202.532999 126.078999) (end 203.708 127.254) (width 0.25) (layer B.Cu) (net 30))
 (segment (start 184.817001 126.078999) (end 202.532999 126.078999) (width 0.25) (layer B.Cu) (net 30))
 (segment (start 183.642 127.254) (end 184.817001 126.078999) (width 0.25) (layer B.Cu) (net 30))
 (segment (start 199.992999 128.429001) (end 201.168 127.254) (width 0.25) (layer F.Cu) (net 29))
 (segment (start 183.077999 128.429001) (end 199.992999 128.429001) (width 0.25) (layer F.Cu) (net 29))
 (segment (start 181.902998 127.254) (end 183.077999 128.429001) (width 0.25) (layer F.Cu) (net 29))
 (segment (start 181.102 127.254) (end 181.902998 127.254) (width 0.25) (layer F.Cu) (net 29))
 (segment (start 202.532999 128.618999) (end 203.708 129.794) (width 0.25) (layer B.Cu) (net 32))
 (segment (start 184.817001 128.618999) (end 202.532999 128.618999) (width 0.25) (layer B.Cu) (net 32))
 (segment (start 183.642 129.794) (end 184.817001 128.618999) (width 0.25) (layer B.Cu) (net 32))
 (segment (start 199.992999 130.969001) (end 201.168 129.794) (width 0.25) (layer F.Cu) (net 31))
 (segment (start 182.277001 130.969001) (end 199.992999 130.969001) (width 0.25) (layer F.Cu) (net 31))
 (segment (start 181.102 129.794) (end 182.277001 130.969001) (width 0.25) (layer F.Cu) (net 31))
 (segment (start 202.532999 131.158999) (end 203.708 132.334) (width 0.25) (layer B.Cu) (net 34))
 (segment (start 184.817001 131.158999) (end 202.532999 131.158999) (width 0.25) (layer B.Cu) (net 34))
 (segment (start 183.642 132.334) (end 184.817001 131.158999) (width 0.25) (layer B.Cu) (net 34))
 (segment (start 199.992999 133.509001) (end 201.168 132.334) (width 0.25) (layer F.Cu) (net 33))
 (segment (start 182.277001 133.509001) (end 199.992999 133.509001) (width 0.25) (layer F.Cu) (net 33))
 (segment (start 181.102 132.334) (end 182.277001 133.509001) (width 0.25) (layer F.Cu) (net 33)))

